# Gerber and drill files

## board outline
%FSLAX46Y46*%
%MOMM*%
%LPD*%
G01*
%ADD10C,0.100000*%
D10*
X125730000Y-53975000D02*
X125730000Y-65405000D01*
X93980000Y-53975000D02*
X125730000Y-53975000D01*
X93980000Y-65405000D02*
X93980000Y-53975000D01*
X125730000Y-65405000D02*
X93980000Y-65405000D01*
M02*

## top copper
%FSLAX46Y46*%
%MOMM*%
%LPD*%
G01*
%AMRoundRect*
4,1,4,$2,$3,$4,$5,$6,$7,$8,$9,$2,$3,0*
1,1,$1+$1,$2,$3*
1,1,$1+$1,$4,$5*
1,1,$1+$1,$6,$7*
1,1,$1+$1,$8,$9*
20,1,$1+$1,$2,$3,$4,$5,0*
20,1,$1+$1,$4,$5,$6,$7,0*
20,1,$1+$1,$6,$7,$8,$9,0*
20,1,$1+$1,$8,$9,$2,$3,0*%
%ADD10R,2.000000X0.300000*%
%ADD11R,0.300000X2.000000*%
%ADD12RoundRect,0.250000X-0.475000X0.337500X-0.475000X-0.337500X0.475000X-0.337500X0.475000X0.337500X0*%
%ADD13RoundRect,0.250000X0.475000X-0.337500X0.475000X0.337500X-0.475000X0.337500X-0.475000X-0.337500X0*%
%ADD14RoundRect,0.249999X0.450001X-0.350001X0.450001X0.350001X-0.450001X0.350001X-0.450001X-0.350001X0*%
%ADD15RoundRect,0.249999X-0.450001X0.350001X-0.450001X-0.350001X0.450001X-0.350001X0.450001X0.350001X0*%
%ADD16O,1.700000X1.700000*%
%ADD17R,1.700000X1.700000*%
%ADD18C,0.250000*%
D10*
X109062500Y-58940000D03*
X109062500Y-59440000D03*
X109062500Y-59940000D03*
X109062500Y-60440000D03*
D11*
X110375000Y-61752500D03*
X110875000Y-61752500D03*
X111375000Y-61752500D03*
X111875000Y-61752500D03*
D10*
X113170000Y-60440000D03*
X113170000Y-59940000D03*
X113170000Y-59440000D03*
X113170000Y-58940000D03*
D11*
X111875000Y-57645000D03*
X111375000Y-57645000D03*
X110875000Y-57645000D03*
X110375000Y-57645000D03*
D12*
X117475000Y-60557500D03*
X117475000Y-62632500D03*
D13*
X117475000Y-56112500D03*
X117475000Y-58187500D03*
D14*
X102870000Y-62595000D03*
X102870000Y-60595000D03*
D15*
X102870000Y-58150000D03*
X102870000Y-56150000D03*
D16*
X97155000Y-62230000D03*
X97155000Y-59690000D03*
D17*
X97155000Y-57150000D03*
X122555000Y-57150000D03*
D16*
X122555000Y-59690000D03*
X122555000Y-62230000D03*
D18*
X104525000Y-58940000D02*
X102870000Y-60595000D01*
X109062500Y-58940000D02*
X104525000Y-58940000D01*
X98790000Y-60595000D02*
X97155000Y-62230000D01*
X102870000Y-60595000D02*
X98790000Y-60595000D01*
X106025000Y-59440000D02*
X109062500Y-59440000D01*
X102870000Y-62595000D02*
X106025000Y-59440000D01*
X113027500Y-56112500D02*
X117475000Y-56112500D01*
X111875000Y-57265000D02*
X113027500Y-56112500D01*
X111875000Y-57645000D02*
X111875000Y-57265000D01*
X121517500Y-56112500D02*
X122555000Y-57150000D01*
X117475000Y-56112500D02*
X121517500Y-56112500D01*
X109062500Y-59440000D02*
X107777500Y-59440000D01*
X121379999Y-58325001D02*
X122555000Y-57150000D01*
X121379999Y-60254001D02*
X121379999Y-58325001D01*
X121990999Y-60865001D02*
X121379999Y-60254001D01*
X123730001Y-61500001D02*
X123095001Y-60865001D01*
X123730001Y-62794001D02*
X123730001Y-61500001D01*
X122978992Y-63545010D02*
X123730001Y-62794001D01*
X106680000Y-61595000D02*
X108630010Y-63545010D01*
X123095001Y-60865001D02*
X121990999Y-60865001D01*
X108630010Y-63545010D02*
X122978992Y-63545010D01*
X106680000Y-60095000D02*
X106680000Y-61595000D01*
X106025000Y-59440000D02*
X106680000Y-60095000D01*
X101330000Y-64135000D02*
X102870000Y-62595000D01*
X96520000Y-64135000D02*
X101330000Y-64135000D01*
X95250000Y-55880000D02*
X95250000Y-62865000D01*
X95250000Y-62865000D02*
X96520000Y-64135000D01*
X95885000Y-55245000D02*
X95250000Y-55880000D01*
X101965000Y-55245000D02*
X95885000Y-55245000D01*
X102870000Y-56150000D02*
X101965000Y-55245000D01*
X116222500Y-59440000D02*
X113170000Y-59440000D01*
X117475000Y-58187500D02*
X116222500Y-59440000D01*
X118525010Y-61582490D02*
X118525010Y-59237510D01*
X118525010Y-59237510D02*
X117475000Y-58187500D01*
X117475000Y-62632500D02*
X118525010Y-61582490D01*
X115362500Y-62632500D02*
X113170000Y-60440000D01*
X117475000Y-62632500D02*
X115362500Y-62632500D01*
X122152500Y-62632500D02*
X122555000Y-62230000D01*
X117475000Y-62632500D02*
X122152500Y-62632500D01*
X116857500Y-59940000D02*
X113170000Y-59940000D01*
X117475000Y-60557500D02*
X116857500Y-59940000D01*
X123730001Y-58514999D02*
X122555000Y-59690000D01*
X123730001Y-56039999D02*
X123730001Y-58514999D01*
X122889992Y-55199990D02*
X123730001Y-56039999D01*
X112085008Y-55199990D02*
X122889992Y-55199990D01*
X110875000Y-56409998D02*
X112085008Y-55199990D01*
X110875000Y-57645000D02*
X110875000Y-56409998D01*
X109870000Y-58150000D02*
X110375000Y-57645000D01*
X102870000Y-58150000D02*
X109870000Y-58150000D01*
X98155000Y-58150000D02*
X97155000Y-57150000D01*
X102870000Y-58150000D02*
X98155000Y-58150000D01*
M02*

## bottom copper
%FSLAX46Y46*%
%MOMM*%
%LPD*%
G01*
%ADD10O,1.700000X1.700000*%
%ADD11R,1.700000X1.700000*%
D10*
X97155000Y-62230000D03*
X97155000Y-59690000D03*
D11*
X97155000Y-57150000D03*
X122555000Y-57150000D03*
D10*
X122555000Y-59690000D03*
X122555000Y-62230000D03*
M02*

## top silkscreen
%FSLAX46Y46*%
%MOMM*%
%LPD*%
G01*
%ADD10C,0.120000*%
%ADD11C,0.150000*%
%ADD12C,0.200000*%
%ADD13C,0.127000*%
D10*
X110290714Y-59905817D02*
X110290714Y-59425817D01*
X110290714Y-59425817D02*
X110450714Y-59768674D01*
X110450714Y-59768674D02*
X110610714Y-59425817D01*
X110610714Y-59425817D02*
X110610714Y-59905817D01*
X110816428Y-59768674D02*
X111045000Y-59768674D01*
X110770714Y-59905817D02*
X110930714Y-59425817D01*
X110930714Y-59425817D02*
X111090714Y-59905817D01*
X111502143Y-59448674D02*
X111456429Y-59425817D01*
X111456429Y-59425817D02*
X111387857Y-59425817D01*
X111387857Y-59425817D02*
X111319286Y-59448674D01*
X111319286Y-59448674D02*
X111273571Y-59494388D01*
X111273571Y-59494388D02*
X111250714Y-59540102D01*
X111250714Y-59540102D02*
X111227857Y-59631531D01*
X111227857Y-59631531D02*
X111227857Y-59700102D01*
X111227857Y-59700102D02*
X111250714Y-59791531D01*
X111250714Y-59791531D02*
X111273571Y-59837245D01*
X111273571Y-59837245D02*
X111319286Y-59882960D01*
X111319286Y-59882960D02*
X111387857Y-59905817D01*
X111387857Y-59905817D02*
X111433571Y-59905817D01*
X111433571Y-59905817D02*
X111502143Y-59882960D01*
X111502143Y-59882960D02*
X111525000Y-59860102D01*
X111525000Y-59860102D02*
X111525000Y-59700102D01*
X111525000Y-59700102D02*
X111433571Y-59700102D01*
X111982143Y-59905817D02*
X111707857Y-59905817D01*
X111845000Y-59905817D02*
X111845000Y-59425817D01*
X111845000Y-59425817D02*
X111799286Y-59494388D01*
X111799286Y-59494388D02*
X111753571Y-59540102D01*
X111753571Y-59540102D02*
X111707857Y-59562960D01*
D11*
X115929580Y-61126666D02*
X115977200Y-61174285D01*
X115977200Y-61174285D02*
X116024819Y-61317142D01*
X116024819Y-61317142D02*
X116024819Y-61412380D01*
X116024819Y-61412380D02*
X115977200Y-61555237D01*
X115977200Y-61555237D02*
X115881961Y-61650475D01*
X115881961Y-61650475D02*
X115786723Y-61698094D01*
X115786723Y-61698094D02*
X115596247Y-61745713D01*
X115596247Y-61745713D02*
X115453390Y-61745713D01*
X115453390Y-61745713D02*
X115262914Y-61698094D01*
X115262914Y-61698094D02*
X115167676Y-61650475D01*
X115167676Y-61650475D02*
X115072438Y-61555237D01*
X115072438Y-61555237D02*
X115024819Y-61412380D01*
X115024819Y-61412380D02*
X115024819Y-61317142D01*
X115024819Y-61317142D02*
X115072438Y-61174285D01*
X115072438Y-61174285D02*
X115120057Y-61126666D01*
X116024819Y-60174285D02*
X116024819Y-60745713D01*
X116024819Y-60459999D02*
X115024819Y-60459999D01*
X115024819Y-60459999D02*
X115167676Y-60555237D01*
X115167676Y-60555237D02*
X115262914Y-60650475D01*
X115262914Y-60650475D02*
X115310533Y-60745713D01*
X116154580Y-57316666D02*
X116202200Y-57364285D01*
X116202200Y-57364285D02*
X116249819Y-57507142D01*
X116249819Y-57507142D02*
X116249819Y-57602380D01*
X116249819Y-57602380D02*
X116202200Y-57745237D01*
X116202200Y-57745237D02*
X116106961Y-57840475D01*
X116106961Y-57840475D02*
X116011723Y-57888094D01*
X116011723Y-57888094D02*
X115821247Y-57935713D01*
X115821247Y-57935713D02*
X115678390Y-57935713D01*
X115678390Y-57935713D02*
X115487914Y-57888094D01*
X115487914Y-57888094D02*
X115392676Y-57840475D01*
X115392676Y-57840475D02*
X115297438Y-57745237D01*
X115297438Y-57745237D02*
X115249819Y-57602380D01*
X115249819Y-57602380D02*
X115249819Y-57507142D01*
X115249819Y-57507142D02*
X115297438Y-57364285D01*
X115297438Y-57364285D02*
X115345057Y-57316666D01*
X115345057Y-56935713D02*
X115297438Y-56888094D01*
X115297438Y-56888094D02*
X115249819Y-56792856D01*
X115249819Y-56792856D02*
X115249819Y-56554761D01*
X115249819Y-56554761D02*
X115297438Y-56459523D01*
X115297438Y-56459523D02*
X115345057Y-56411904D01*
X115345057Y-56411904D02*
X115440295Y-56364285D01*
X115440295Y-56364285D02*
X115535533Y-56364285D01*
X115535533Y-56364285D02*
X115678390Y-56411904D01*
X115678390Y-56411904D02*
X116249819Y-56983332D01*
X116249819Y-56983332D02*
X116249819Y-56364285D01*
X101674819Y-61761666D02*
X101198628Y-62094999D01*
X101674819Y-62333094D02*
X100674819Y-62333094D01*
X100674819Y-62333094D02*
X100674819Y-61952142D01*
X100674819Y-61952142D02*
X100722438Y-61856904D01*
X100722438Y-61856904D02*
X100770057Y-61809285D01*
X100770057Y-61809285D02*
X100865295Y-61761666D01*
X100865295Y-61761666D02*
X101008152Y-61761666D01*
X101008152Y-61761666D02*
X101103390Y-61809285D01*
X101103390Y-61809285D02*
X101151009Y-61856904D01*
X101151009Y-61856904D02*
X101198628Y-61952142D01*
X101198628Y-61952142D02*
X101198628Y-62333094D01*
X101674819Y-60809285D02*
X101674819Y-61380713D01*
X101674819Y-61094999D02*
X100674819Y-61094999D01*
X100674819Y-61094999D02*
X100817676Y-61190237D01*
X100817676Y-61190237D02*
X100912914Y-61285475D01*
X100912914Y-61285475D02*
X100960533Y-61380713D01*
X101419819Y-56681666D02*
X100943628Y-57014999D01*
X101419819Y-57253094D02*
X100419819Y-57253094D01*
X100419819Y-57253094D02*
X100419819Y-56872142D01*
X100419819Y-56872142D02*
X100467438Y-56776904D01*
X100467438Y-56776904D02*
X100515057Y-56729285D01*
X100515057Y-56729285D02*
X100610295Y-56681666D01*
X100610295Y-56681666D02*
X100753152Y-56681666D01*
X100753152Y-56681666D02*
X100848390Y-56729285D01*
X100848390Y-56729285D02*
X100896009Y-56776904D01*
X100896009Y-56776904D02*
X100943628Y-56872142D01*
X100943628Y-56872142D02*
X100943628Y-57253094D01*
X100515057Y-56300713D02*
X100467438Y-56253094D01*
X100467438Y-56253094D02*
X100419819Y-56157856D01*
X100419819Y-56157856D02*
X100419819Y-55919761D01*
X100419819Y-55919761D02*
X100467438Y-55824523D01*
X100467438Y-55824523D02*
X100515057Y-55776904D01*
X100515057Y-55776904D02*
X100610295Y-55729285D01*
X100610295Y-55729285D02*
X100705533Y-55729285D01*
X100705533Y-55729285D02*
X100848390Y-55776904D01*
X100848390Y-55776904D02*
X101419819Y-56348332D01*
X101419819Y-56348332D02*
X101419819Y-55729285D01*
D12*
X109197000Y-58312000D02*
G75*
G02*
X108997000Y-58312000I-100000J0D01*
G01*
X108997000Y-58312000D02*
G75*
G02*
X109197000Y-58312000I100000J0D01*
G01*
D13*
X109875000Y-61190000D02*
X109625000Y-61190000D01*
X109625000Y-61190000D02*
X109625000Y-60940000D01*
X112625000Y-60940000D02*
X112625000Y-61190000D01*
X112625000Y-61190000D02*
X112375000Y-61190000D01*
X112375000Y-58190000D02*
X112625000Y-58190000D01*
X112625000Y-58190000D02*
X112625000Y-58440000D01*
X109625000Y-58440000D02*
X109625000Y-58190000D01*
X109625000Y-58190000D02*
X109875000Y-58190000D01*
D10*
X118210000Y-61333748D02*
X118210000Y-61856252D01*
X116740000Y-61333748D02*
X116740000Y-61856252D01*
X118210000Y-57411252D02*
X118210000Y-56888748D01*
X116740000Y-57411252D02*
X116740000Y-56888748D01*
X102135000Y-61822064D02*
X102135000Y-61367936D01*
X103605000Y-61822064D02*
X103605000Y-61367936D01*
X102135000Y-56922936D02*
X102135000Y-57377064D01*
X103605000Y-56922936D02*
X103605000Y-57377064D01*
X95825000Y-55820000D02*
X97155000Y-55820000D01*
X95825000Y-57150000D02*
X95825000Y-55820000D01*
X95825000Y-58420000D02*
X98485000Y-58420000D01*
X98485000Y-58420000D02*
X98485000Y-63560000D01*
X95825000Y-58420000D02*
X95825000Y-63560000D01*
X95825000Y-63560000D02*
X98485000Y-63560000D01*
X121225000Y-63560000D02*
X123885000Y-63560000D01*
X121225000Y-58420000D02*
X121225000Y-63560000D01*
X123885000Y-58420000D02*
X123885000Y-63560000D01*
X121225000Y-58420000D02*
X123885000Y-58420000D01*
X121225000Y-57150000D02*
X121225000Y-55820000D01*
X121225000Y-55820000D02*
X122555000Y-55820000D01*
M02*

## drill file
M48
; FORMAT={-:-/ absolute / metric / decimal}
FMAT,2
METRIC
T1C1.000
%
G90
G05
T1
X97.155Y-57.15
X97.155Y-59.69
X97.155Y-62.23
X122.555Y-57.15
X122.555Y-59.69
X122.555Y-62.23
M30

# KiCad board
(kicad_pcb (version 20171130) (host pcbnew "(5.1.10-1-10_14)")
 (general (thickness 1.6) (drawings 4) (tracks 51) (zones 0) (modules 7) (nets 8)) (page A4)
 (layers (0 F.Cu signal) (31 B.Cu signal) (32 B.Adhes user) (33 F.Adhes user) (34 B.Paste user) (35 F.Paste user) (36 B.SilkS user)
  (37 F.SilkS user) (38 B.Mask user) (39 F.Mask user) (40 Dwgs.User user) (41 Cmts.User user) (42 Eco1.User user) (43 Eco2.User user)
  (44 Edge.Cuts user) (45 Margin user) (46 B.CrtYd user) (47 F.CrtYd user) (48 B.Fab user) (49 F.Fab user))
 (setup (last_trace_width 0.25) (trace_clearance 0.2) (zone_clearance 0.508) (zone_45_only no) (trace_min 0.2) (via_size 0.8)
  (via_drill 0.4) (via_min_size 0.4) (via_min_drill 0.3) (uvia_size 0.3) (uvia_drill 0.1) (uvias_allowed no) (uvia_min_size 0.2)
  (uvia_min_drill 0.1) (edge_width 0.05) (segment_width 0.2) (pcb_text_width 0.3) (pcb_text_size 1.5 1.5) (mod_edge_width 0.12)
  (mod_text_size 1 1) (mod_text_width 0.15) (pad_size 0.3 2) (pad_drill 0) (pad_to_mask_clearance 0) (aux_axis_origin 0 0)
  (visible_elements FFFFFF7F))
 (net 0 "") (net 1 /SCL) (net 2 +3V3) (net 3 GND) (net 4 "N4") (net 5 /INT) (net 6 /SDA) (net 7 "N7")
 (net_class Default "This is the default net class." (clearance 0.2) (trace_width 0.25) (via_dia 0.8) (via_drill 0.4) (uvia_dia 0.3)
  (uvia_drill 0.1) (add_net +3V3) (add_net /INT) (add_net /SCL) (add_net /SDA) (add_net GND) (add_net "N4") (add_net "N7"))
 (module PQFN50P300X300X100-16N (layer F.Cu) (at 111.125 59.69)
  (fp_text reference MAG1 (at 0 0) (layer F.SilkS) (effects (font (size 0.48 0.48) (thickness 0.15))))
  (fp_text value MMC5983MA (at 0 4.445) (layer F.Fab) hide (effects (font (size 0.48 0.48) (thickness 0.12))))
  (fp_circle (center -2.028 -1.378) (end -1.928 -1.378) (layer F.SilkS) (width 0.2))
  (fp_line (start -1.25 1.5) (end -1.5 1.5) (layer F.SilkS) (width 0.127))
  (fp_line (start -1.5 1.5) (end -1.5 1.25) (layer F.SilkS) (width 0.127))
  (fp_line (start 1.5 1.25) (end 1.5 1.5) (layer F.SilkS) (width 0.127))
  (fp_line (start 1.5 1.5) (end 1.25 1.5) (layer F.SilkS) (width 0.127))
  (fp_line (start 1.25 -1.5) (end 1.5 -1.5) (layer F.SilkS) (width 0.127))
  (fp_line (start 1.5 -1.5) (end 1.5 -1.25) (layer F.SilkS) (width 0.127))
  (fp_line (start -1.5 -1.25) (end -1.5 -1.5) (layer F.SilkS) (width 0.127))
  (fp_line (start -1.5 -1.5) (end -1.25 -1.5) (layer F.SilkS) (width 0.127))
  (pad 1 smd rect (at -2.0625 -0.75) (size 2 0.3) (layers F.Cu F.Paste F.Mask) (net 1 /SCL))
  (pad 2 smd rect (at -2.0625 -0.25) (size 2 0.3) (layers F.Cu F.Paste F.Mask) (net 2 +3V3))
  (pad 3 smd rect (at -2.0625 0.25) (size 2 0.3) (layers F.Cu F.Paste F.Mask))
  (pad 4 smd rect (at -2.0625 0.75) (size 2 0.3) (layers F.Cu F.Paste F.Mask))
  (pad 5 smd rect (at -0.75 2.0625) (size 0.3 2) (layers F.Cu F.Paste F.Mask))
  (pad 6 smd rect (at -0.25 2.0625) (size 0.3 2) (layers F.Cu F.Paste F.Mask))
  (pad 7 smd rect (at 0.25 2.0625) (size 0.3 2) (layers F.Cu F.Paste F.Mask))
  (pad 8 smd rect (at 0.75 2.0625) (size 0.3 2) (layers F.Cu F.Paste F.Mask))
  (pad 9 smd rect (at 2.045 0.75) (size 2 0.3) (layers F.Cu F.Paste F.Mask) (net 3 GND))
  (pad 10 smd rect (at 2.045 0.25) (size 2 0.3) (layers F.Cu F.Paste F.Mask) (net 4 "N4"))
  (pad 11 smd rect (at 2.045 -0.25) (size 2 0.3) (layers F.Cu F.Paste F.Mask) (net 3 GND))
  (pad 12 smd rect (at 2.045 -0.75) (size 2 0.3) (layers F.Cu F.Paste F.Mask))
  (pad 13 smd rect (at 0.75 -2.045) (size 0.3 2) (layers F.Cu F.Paste F.Mask) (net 2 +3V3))
  (pad 14 smd rect (at 0.25 -2.045) (size 0.3 2) (layers F.Cu F.Paste F.Mask))
  (pad 15 smd rect (at -0.25 -2.045) (size 0.3 2) (layers F.Cu F.Paste F.Mask) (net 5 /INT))
  (pad 16 smd rect (at -0.75 -2.045) (size 0.3 2) (layers F.Cu F.Paste F.Mask) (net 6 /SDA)))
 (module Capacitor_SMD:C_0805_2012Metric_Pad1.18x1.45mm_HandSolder (layer F.Cu) (at 117.475 61.595 270)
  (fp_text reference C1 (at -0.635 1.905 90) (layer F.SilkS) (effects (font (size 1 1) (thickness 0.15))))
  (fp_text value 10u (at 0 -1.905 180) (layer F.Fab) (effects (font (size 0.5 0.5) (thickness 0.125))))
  (fp_line (start -0.261252 -0.735) (end 0.261252 -0.735) (layer F.SilkS) (width 0.12))
  (fp_line (start -0.261252 0.735) (end 0.261252 0.735) (layer F.SilkS) (width 0.12))
  (pad 1 smd roundrect (at -1.0375 0 270) (size 1.175 1.45) (layers F.Cu F.Paste F.Mask) (roundrect_rratio 0.2127659574468085) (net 4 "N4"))
  (pad 2 smd roundrect (at 1.0375 0 270) (size 1.175 1.45) (layers F.Cu F.Paste F.Mask) (roundrect_rratio 0.2127659574468085) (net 3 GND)))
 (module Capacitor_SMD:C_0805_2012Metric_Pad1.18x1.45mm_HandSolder (layer F.Cu) (at 117.475 57.15 90)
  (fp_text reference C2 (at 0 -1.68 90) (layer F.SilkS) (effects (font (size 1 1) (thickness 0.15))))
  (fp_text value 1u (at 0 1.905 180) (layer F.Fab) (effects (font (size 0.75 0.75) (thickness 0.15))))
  (fp_line (start -0.261252 0.735) (end 0.261252 0.735) (layer F.SilkS) (width 0.12))
  (fp_line (start -0.261252 -0.735) (end 0.261252 -0.735) (layer F.SilkS) (width 0.12))
  (pad 2 smd roundrect (at 1.0375 0 90) (size 1.175 1.45) (layers F.Cu F.Paste F.Mask) (roundrect_rratio 0.2127659574468085) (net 2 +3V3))
  (pad 1 smd roundrect (at -1.0375 0 90) (size 1.175 1.45) (layers F.Cu F.Paste F.Mask) (roundrect_rratio 0.2127659574468085) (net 3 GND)))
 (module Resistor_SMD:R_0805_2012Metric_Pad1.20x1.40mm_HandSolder (layer F.Cu) (at 102.87 61.595 90)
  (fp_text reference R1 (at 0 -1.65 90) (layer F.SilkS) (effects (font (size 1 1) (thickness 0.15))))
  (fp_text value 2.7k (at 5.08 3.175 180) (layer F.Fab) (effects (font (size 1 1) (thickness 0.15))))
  (fp_line (start -0.227064 -0.735) (end 0.227064 -0.735) (layer F.SilkS) (width 0.12))
  (fp_line (start -0.227064 0.735) (end 0.227064 0.735) (layer F.SilkS) (width 0.12))
  (pad 1 smd roundrect (at -1 0 90) (size 1.2 1.4) (layers F.Cu F.Paste F.Mask) (roundrect_rratio 0.2083325) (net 2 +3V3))
  (pad 2 smd roundrect (at 1 0 90) (size 1.2 1.4) (layers F.Cu F.Paste F.Mask) (roundrect_rratio 0.2083325) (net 1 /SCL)))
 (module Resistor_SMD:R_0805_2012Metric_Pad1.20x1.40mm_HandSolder (layer F.Cu) (at 102.87 57.15 270)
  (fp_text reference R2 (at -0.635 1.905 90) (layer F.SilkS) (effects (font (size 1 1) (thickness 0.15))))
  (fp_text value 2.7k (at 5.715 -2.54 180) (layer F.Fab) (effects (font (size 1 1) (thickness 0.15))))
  (fp_line (start -0.227064 0.735) (end 0.227064 0.735) (layer F.SilkS) (width 0.12))
  (fp_line (start -0.227064 -0.735) (end 0.227064 -0.735) (layer F.SilkS) (width 0.12))
  (pad 2 smd roundrect (at 1 0 270) (size 1.2 1.4) (layers F.Cu F.Paste F.Mask) (roundrect_rratio 0.2083325) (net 6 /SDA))
  (pad 1 smd roundrect (at -1 0 270) (size 1.2 1.4) (layers F.Cu F.Paste F.Mask) (roundrect_rratio 0.2083325) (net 2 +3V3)))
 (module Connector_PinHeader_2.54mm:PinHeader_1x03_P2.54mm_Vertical (layer F.Cu) (at 97.155 57.15)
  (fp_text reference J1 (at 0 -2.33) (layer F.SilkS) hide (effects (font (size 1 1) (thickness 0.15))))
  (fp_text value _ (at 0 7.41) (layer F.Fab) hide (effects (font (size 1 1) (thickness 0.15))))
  (fp_line (start -1.33 -1.33) (end 0 -1.33) (layer F.SilkS) (width 0.12))
  (fp_line (start -1.33 0) (end -1.33 -1.33) (layer F.SilkS) (width 0.12))
  (fp_line (start -1.33 1.27) (end 1.33 1.27) (layer F.SilkS) (width 0.12))
  (fp_line (start 1.33 1.27) (end 1.33 6.41) (layer F.SilkS) (width 0.12))
  (fp_line (start -1.33 1.27) (end -1.33 6.41) (layer F.SilkS) (width 0.12))
  (fp_line (start -1.33 6.41) (end 1.33 6.41) (layer F.SilkS) (width 0.12))
  (pad 3 thru_hole oval (at 0 5.08) (size 1.7 1.7) (drill 1) (layers *.Cu *.Mask) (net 1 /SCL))
  (pad 2 thru_hole oval (at 0 2.54) (size 1.7 1.7) (drill 1) (layers *.Cu *.Mask) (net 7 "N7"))
  (pad 1 thru_hole rect (at 0 0) (size 1.7 1.7) (drill 1) (layers *.Cu *.Mask) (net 6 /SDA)))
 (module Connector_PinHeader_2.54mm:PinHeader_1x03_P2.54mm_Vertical (layer F.Cu) (at 122.555 57.15)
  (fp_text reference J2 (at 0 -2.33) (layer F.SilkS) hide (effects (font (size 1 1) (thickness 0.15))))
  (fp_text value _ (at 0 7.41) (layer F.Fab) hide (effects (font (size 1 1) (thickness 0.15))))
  (fp_line (start -1.33 6.41) (end 1.33 6.41) (layer F.SilkS) (width 0.12))
  (fp_line (start -1.33 1.27) (end -1.33 6.41) (layer F.SilkS) (width 0.12))
  (fp_line (start 1.33 1.27) (end 1.33 6.41) (layer F.SilkS) (width 0.12))
  (fp_line (start -1.33 1.27) (end 1.33 1.27) (layer F.SilkS) (width 0.12))
  (fp_line (start -1.33 0) (end -1.33 -1.33) (layer F.SilkS) (width 0.12))
  (fp_line (start -1.33 -1.33) (end 0 -1.33) (layer F.SilkS) (width 0.12))
  (pad 1 thru_hole rect (at 0 0) (size 1.7 1.7) (drill 1) (layers *.Cu *.Mask) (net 2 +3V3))
  (pad 2 thru_hole oval (at 0 2.54) (size 1.7 1.7) (drill 1) (layers *.Cu *.Mask) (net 5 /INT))
  (pad 3 thru_hole oval (at 0 5.08) (size 1.7 1.7) (drill 1) (layers *.Cu *.Mask) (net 3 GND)))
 (gr_line (start 125.73 53.975) (end 125.73 65.405) (layer Edge.Cuts) (width 0.1))
 (gr_line (start 93.98 53.975) (end 125.73 53.975) (layer Edge.Cuts) (width 0.1))
 (gr_line (start 93.98 65.405) (end 93.98 53.975) (layer Edge.Cuts) (width 0.1))
 (gr_line (start 125.73 65.405) (end 93.98 65.405) (layer Edge.Cuts) (width 0.1))
 (segment (start 104.525 58.94) (end 102.87 60.595) (width 0.25) (layer F.Cu) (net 1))
 (segment (start 109.0625 58.94) (end 104.525 58.94) (width 0.25) (layer F.Cu) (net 1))
 (segment (start 98.79 60.595) (end 97.155 62.23) (width 0.25) (layer F.Cu) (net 1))
 (segment (start 102.87 60.595) (end 98.79 60.595) (width 0.25) (layer F.Cu) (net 1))
 (segment (start 106.025 59.44) (end 109.0625 59.44) (width 0.25) (layer F.Cu) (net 2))
 (segment (start 102.87 62.595) (end 106.025 59.44) (width 0.25) (layer F.Cu) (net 2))
 (segment (start 113.0275 56.1125) (end 117.475 56.1125) (width 0.25) (layer F.Cu) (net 2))
 (segment (start 111.875 57.265) (end 113.0275 56.1125) (width 0.25) (layer F.Cu) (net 2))
 (segment (start 111.875 57.645) (end 111.875 57.265) (width 0.25) (layer F.Cu) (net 2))
 (segment (start 121.5175 56.1125) (end 122.555 57.15) (width 0.25) (layer F.Cu) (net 2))
 (segment (start 117.475 56.1125) (end 121.5175 56.1125) (width 0.25) (layer F.Cu) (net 2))
 (segment (start 109.0625 59.44) (end 107.7775 59.44) (width 0.25) (layer F.Cu) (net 2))
 (segment (start 121.379999 58.325001) (end 122.555 57.15) (width 0.25) (layer F.Cu) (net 2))
 (segment (start 121.379999 60.254001) (end 121.379999 58.325001) (width 0.25) (layer F.Cu) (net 2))
 (segment (start 121.990999 60.865001) (end 121.379999 60.254001) (width 0.25) (layer F.Cu) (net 2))
 (segment (start 123.730001 61.500001) (end 123.095001 60.865001) (width 0.25) (layer F.Cu) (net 2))
 (segment (start 123.730001 62.794001) (end 123.730001 61.500001) (width 0.25) (layer F.Cu) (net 2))
 (segment (start 122.978992 63.54501) (end 123.730001 62.794001) (width 0.25) (layer F.Cu) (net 2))
 (segment (start 106.68 61.595) (end 108.63001 63.54501) (width 0.25) (layer F.Cu) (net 2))
 (segment (start 123.095001 60.865001) (end 121.990999 60.865001) (width 0.25) (layer F.Cu) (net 2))
 (segment (start 108.63001 63.54501) (end 122.978992 63.54501) (width 0.25) (layer F.Cu) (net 2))
 (segment (start 106.68 60.095) (end 106.68 61.595) (width 0.25) (layer F.Cu) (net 2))
 (segment (start 106.025 59.44) (end 106.68 60.095) (width 0.25) (layer F.Cu) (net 2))
 (segment (start 101.33 64.135) (end 102.87 62.595) (width 0.25) (layer F.Cu) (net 2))
 (segment (start 96.52 64.135) (end 101.33 64.135) (width 0.25) (layer F.Cu) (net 2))
 (segment (start 95.25 55.88) (end 95.25 62.865) (width 0.25) (layer F.Cu) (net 2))
 (segment (start 95.25 62.865) (end 96.52 64.135) (width 0.25) (layer F.Cu) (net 2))
 (segment (start 95.885 55.245) (end 95.25 55.88) (width 0.25) (layer F.Cu) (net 2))
 (segment (start 101.965 55.245) (end 95.885 55.245) (width 0.25) (layer F.Cu) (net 2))
 (segment (start 102.87 56.15) (end 101.965 55.245) (width 0.25) (layer F.Cu) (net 2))
 (segment (start 116.2225 59.44) (end 113.17 59.44) (width 0.25) (layer F.Cu) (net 3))
 (segment (start 117.475 58.1875) (end 116.2225 59.44) (width 0.25) (layer F.Cu) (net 3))
 (segment (start 118.52501 61.58249) (end 118.52501 59.23751) (width 0.25) (layer F.Cu) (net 3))
 (segment (start 118.52501 59.23751) (end 117.475 58.1875) (width 0.25) (layer F.Cu) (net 3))
 (segment (start 117.475 62.6325) (end 118.52501 61.58249) (width 0.25) (layer F.Cu) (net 3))
 (segment (start 115.3625 62.6325) (end 113.17 60.44) (width 0.25) (layer F.Cu) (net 3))
 (segment (start 117.475 62.6325) (end 115.3625 62.6325) (width 0.25) (layer F.Cu) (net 3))
 (segment (start 122.1525 62.6325) (end 122.555 62.23) (width 0.25) (layer F.Cu) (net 3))
 (segment (start 117.475 62.6325) (end 122.1525 62.6325) (width 0.25) (layer F.Cu) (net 3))
 (segment (start 116.8575 59.94) (end 113.17 59.94) (width 0.25) (layer F.Cu) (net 4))
 (segment (start 117.475 60.5575) (end 116.8575 59.94) (width 0.25) (layer F.Cu) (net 4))
 (segment (start 123.730001 58.514999) (end 122.555 59.69) (width 0.25) (layer F.Cu) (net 5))
 (segment (start 123.730001 56.039999) (end 123.730001 58.514999) (width 0.25) (layer F.Cu) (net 5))
 (segment (start 122.889992 55.19999) (end 123.730001 56.039999) (width 0.25) (layer F.Cu) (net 5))
 (segment (start 112.085008 55.19999) (end 122.889992 55.19999) (width 0.25) (layer F.Cu) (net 5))
 (segment (start 110.875 56.409998) (end 112.085008 55.19999) (width 0.25) (layer F.Cu) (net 5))
 (segment (start 110.875 57.645) (end 110.875 56.409998) (width 0.25) (layer F.Cu) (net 5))
 (segment (start 109.87 58.15) (end 110.375 57.645) (width 0.25) (layer F.Cu) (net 6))
 (segment (start 102.87 58.15) (end 109.87 58.15) (width 0.25) (layer F.Cu) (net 6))
 (segment (start 98.155 58.15) (end 97.155 57.15) (width 0.25) (layer F.Cu) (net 6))
 (segment (start 102.87 58.15) (end 98.155 58.15) (width 0.25) (layer F.Cu) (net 6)))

